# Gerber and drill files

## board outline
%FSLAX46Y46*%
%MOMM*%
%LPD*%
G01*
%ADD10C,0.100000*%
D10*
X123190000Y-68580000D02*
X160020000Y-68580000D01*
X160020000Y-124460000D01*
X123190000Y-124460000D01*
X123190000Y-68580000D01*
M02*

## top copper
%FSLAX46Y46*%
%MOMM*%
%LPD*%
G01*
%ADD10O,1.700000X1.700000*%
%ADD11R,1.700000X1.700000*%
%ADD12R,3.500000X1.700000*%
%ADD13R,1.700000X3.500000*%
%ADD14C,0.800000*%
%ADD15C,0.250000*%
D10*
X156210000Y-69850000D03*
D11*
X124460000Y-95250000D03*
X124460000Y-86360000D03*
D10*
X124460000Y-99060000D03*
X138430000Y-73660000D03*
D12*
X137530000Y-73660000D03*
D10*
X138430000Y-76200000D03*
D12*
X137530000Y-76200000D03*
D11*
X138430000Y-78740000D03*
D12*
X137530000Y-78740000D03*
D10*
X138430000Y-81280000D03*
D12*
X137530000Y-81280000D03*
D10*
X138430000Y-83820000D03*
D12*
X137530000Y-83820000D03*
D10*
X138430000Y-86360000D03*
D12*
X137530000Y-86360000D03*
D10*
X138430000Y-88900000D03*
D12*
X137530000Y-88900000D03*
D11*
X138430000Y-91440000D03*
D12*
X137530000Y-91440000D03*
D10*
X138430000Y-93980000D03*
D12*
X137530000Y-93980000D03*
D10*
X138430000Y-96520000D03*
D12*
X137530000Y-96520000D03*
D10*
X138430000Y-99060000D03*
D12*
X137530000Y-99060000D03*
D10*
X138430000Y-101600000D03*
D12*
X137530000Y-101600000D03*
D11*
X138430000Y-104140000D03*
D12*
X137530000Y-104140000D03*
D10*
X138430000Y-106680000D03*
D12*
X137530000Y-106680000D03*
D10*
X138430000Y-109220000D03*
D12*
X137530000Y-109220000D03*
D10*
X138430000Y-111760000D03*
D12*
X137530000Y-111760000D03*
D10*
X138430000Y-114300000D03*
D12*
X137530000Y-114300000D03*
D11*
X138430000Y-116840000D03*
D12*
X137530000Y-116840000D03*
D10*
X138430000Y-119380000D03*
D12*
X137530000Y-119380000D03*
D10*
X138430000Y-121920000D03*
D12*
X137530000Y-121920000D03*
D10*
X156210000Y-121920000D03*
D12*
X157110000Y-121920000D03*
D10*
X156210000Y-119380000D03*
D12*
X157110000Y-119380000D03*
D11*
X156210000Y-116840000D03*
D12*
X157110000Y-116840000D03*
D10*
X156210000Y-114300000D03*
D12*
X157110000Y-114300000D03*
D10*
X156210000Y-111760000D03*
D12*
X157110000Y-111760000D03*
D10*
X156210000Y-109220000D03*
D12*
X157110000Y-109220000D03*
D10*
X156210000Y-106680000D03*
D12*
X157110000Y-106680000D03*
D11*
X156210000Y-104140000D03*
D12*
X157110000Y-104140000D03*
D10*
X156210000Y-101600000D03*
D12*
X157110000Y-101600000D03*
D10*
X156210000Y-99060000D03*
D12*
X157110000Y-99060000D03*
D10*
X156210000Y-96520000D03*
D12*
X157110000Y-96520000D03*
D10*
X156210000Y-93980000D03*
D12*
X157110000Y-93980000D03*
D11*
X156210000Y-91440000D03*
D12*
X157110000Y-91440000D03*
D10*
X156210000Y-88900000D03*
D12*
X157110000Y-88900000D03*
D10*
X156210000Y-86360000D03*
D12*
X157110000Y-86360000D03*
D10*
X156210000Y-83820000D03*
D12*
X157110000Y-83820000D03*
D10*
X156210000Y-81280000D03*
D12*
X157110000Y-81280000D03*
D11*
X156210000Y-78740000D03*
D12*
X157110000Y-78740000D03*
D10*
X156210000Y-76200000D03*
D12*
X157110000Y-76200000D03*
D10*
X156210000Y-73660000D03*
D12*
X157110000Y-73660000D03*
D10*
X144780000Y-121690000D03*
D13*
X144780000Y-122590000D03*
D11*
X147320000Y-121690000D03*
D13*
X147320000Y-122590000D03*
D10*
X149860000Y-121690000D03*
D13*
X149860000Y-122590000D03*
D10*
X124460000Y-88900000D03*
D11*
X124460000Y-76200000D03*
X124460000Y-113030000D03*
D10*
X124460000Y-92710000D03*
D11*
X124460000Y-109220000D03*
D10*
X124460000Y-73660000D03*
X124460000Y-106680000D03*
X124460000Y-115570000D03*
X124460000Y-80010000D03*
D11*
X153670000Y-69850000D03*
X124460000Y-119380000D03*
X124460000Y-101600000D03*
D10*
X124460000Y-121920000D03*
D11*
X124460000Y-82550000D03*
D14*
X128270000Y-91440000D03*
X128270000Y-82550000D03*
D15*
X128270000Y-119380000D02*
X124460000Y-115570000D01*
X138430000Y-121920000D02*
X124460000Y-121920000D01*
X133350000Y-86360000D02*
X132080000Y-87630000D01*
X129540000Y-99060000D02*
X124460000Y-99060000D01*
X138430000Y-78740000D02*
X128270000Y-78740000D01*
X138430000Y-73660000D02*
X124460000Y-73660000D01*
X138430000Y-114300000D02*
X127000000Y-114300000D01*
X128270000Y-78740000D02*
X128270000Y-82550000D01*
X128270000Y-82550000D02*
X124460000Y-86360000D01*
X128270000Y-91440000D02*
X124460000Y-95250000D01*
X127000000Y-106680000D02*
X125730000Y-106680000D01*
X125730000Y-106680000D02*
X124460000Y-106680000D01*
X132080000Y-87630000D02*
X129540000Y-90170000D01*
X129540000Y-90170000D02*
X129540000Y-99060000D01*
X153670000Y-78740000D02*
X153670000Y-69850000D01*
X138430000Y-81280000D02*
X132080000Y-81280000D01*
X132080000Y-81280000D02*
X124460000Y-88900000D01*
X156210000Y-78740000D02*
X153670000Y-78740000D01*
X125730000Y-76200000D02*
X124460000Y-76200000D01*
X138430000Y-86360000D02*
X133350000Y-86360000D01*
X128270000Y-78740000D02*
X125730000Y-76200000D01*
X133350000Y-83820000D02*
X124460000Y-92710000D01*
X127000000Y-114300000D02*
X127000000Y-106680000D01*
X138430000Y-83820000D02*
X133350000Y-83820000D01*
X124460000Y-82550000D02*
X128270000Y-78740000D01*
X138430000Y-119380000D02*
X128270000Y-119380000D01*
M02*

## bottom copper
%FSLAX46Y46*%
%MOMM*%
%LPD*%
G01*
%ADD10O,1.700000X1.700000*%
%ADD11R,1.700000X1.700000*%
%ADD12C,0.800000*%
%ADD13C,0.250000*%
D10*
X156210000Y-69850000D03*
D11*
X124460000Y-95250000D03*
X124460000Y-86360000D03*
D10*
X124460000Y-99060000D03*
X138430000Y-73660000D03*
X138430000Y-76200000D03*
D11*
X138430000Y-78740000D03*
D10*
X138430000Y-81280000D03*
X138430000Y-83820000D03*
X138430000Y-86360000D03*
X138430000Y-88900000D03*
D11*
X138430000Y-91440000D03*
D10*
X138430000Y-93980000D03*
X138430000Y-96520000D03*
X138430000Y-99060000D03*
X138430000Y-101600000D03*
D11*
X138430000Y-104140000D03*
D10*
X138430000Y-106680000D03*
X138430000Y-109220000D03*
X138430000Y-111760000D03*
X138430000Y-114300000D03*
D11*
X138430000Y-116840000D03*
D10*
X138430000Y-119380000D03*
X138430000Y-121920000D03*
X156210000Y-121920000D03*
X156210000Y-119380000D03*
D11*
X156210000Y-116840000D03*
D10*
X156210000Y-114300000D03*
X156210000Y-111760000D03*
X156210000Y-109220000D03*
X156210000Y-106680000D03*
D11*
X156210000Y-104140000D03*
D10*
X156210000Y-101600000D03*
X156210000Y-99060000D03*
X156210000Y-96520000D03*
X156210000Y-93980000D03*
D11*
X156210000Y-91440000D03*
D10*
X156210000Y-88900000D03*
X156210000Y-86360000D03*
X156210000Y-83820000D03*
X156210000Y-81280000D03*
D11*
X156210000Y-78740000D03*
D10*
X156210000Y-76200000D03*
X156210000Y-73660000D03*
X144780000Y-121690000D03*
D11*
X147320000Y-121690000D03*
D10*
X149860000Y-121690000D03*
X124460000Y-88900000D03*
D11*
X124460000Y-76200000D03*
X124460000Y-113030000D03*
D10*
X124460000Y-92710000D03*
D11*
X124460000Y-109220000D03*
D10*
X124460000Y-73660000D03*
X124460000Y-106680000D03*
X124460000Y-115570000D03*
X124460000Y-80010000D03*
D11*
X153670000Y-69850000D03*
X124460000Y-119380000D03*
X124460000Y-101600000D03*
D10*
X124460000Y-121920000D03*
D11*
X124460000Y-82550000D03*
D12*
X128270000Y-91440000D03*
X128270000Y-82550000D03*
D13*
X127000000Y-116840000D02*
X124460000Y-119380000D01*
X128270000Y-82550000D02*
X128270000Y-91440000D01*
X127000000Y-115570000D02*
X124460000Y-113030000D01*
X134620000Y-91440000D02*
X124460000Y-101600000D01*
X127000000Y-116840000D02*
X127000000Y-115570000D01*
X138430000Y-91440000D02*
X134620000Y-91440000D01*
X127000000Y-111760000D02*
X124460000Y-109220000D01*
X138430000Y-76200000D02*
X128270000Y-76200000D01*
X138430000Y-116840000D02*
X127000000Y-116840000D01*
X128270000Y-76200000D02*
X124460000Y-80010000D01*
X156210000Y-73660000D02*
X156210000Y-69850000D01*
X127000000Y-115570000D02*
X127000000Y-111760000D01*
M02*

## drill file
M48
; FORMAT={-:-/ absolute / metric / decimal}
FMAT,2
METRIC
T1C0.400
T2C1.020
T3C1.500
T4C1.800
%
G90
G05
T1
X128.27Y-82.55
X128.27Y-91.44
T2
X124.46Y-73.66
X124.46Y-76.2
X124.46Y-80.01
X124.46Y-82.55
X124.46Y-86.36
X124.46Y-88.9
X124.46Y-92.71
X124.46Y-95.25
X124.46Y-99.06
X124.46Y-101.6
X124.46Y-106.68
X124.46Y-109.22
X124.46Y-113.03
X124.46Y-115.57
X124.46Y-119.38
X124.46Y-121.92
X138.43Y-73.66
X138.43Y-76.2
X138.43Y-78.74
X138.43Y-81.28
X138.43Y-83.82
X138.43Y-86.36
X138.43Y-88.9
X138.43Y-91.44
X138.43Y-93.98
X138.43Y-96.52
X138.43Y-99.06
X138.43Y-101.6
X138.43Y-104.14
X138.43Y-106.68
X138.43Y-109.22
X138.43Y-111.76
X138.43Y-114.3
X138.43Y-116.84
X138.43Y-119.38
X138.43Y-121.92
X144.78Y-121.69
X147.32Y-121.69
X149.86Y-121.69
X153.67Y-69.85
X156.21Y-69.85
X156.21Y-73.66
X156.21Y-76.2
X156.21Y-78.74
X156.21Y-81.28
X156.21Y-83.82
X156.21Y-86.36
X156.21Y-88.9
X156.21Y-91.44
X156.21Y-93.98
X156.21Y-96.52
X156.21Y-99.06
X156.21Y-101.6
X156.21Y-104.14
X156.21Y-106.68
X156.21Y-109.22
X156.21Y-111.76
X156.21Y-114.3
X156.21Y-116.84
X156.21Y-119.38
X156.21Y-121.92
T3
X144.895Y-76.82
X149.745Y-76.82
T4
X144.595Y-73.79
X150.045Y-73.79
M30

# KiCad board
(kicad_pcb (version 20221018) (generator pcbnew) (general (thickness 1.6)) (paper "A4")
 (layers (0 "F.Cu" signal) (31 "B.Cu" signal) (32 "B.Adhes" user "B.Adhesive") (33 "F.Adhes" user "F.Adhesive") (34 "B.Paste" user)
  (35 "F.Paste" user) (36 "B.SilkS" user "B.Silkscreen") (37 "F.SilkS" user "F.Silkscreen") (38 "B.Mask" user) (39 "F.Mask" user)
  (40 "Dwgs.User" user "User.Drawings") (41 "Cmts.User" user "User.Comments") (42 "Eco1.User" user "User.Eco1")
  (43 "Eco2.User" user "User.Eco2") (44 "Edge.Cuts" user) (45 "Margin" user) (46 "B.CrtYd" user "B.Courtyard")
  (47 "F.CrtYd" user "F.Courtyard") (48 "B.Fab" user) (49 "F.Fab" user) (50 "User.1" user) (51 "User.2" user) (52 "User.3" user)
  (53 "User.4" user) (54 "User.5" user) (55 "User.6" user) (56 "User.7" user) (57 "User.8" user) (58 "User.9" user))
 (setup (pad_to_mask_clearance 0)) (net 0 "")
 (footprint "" (layer "F.Cu") (at 156.21 69.85)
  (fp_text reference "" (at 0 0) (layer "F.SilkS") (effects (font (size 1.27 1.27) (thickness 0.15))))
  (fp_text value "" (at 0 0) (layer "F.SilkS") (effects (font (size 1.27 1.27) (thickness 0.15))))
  (pad "39" thru_hole oval (at 0 0) (size 1.7 1.7) (drill 1.02) (layers "*.Cu" "*.Mask")))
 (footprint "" (layer "F.Cu") (at 124.46 95.25)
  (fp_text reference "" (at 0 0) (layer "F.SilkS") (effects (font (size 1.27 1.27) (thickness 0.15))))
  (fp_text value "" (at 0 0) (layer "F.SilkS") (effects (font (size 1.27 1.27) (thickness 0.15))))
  (pad "3" thru_hole rect (at 0 0) (size 1.7 1.7) (drill 1.02) (layers "*.Cu" "*.Mask")))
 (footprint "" (layer "F.Cu") (at 124.46 86.36)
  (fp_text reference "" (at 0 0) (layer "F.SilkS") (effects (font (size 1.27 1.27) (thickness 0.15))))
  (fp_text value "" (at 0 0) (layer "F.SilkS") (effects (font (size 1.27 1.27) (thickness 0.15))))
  (pad "3" thru_hole rect (at 0 0) (size 1.7 1.7) (drill 1.02) (layers "*.Cu" "*.Mask")))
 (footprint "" (layer "F.Cu") (at 124.46 99.06)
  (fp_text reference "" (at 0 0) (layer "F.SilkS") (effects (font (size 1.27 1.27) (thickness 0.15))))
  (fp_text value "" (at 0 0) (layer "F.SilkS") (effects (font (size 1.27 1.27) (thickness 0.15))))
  (pad "6" thru_hole oval (at 0 0) (size 1.7 1.7) (drill 1.02) (layers "*.Cu" "*.Mask")))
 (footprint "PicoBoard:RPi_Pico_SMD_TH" (layer "F.Cu") (at 147.32 97.79)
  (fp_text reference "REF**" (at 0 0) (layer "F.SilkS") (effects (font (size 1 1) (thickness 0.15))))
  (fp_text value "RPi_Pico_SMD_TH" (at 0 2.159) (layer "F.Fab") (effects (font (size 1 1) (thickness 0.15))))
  (pad "" np_thru_hole oval (at -2.725 -24) (size 1.8 1.8) (drill 1.8) (layers "*.Cu" "*.Mask"))
  (pad "" np_thru_hole oval (at -2.425 -20.97) (size 1.5 1.5) (drill 1.5) (layers "*.Cu" "*.Mask"))
  (pad "" np_thru_hole oval (at 2.425 -20.97) (size 1.5 1.5) (drill 1.5) (layers "*.Cu" "*.Mask"))
  (pad "" np_thru_hole oval (at 2.725 -24) (size 1.8 1.8) (drill 1.8) (layers "*.Cu" "*.Mask"))
  (pad "1" thru_hole oval (at -8.89 -24.13) (size 1.7 1.7) (drill 1.02) (layers "*.Cu" "*.Mask"))
  (pad "1" smd rect (at -8.89 -24.13) (size 3.5 1.7) (drill (offset -0.9 0)) (layers "F.Cu" "F.Mask"))
  (pad "2" thru_hole oval (at -8.89 -21.59) (size 1.7 1.7) (drill 1.02) (layers "*.Cu" "*.Mask"))
  (pad "2" smd rect (at -8.89 -21.59) (size 3.5 1.7) (drill (offset -0.9 0)) (layers "F.Cu" "F.Mask"))
  (pad "3" thru_hole rect (at -8.89 -19.05) (size 1.7 1.7) (drill 1.02) (layers "*.Cu" "*.Mask"))
  (pad "3" smd rect (at -8.89 -19.05) (size 3.5 1.7) (drill (offset -0.9 0)) (layers "F.Cu" "F.Mask"))
  (pad "4" thru_hole oval (at -8.89 -16.51) (size 1.7 1.7) (drill 1.02) (layers "*.Cu" "*.Mask"))
  (pad "4" smd rect (at -8.89 -16.51) (size 3.5 1.7) (drill (offset -0.9 0)) (layers "F.Cu" "F.Mask"))
  (pad "5" thru_hole oval (at -8.89 -13.97) (size 1.7 1.7) (drill 1.02) (layers "*.Cu" "*.Mask"))
  (pad "5" smd rect (at -8.89 -13.97) (size 3.5 1.7) (drill (offset -0.9 0)) (layers "F.Cu" "F.Mask"))
  (pad "6" thru_hole oval (at -8.89 -11.43) (size 1.7 1.7) (drill 1.02) (layers "*.Cu" "*.Mask"))
  (pad "6" smd rect (at -8.89 -11.43) (size 3.5 1.7) (drill (offset -0.9 0)) (layers "F.Cu" "F.Mask"))
  (pad "7" thru_hole oval (at -8.89 -8.89) (size 1.7 1.7) (drill 1.02) (layers "*.Cu" "*.Mask"))
  (pad "7" smd rect (at -8.89 -8.89) (size 3.5 1.7) (drill (offset -0.9 0)) (layers "F.Cu" "F.Mask"))
  (pad "8" thru_hole rect (at -8.89 -6.35) (size 1.7 1.7) (drill 1.02) (layers "*.Cu" "*.Mask"))
  (pad "8" smd rect (at -8.89 -6.35) (size 3.5 1.7) (drill (offset -0.9 0)) (layers "F.Cu" "F.Mask"))
  (pad "9" thru_hole oval (at -8.89 -3.81) (size 1.7 1.7) (drill 1.02) (layers "*.Cu" "*.Mask"))
  (pad "9" smd rect (at -8.89 -3.81) (size 3.5 1.7) (drill (offset -0.9 0)) (layers "F.Cu" "F.Mask"))
  (pad "10" thru_hole oval (at -8.89 -1.27) (size 1.7 1.7) (drill 1.02) (layers "*.Cu" "*.Mask"))
  (pad "10" smd rect (at -8.89 -1.27) (size 3.5 1.7) (drill (offset -0.9 0)) (layers "F.Cu" "F.Mask"))
  (pad "11" thru_hole oval (at -8.89 1.27) (size 1.7 1.7) (drill 1.02) (layers "*.Cu" "*.Mask"))
  (pad "11" smd rect (at -8.89 1.27) (size 3.5 1.7) (drill (offset -0.9 0)) (layers "F.Cu" "F.Mask"))
  (pad "12" thru_hole oval (at -8.89 3.81) (size 1.7 1.7) (drill 1.02) (layers "*.Cu" "*.Mask"))
  (pad "12" smd rect (at -8.89 3.81) (size 3.5 1.7) (drill (offset -0.9 0)) (layers "F.Cu" "F.Mask"))
  (pad "13" thru_hole rect (at -8.89 6.35) (size 1.7 1.7) (drill 1.02) (layers "*.Cu" "*.Mask"))
  (pad "13" smd rect (at -8.89 6.35) (size 3.5 1.7) (drill (offset -0.9 0)) (layers "F.Cu" "F.Mask"))
  (pad "14" thru_hole oval (at -8.89 8.89) (size 1.7 1.7) (drill 1.02) (layers "*.Cu" "*.Mask"))
  (pad "14" smd rect (at -8.89 8.89) (size 3.5 1.7) (drill (offset -0.9 0)) (layers "F.Cu" "F.Mask"))
  (pad "15" thru_hole oval (at -8.89 11.43) (size 1.7 1.7) (drill 1.02) (layers "*.Cu" "*.Mask"))
  (pad "15" smd rect (at -8.89 11.43) (size 3.5 1.7) (drill (offset -0.9 0)) (layers "F.Cu" "F.Mask"))
  (pad "16" thru_hole oval (at -8.89 13.97) (size 1.7 1.7) (drill 1.02) (layers "*.Cu" "*.Mask"))
  (pad "16" smd rect (at -8.89 13.97) (size 3.5 1.7) (drill (offset -0.9 0)) (layers "F.Cu" "F.Mask"))
  (pad "17" thru_hole oval (at -8.89 16.51) (size 1.7 1.7) (drill 1.02) (layers "*.Cu" "*.Mask"))
  (pad "17" smd rect (at -8.89 16.51) (size 3.5 1.7) (drill (offset -0.9 0)) (layers "F.Cu" "F.Mask"))
  (pad "18" thru_hole rect (at -8.89 19.05) (size 1.7 1.7) (drill 1.02) (layers "*.Cu" "*.Mask"))
  (pad "18" smd rect (at -8.89 19.05) (size 3.5 1.7) (drill (offset -0.9 0)) (layers "F.Cu" "F.Mask"))
  (pad "19" thru_hole oval (at -8.89 21.59) (size 1.7 1.7) (drill 1.02) (layers "*.Cu" "*.Mask"))
  (pad "19" smd rect (at -8.89 21.59) (size 3.5 1.7) (drill (offset -0.9 0)) (layers "F.Cu" "F.Mask"))
  (pad "20" thru_hole oval (at -8.89 24.13) (size 1.7 1.7) (drill 1.02) (layers "*.Cu" "*.Mask"))
  (pad "20" smd rect (at -8.89 24.13) (size 3.5 1.7) (drill (offset -0.9 0)) (layers "F.Cu" "F.Mask"))
  (pad "21" thru_hole oval (at 8.89 24.13) (size 1.7 1.7) (drill 1.02) (layers "*.Cu" "*.Mask"))
  (pad "21" smd rect (at 8.89 24.13) (size 3.5 1.7) (drill (offset 0.9 0)) (layers "F.Cu" "F.Mask"))
  (pad "22" thru_hole oval (at 8.89 21.59) (size 1.7 1.7) (drill 1.02) (layers "*.Cu" "*.Mask"))
  (pad "22" smd rect (at 8.89 21.59) (size 3.5 1.7) (drill (offset 0.9 0)) (layers "F.Cu" "F.Mask"))
  (pad "23" thru_hole rect (at 8.89 19.05) (size 1.7 1.7) (drill 1.02) (layers "*.Cu" "*.Mask"))
  (pad "23" smd rect (at 8.89 19.05) (size 3.5 1.7) (drill (offset 0.9 0)) (layers "F.Cu" "F.Mask"))
  (pad "24" thru_hole oval (at 8.89 16.51) (size 1.7 1.7) (drill 1.02) (layers "*.Cu" "*.Mask"))
  (pad "24" smd rect (at 8.89 16.51) (size 3.5 1.7) (drill (offset 0.9 0)) (layers "F.Cu" "F.Mask"))
  (pad "25" thru_hole oval (at 8.89 13.97) (size 1.7 1.7) (drill 1.02) (layers "*.Cu" "*.Mask"))
  (pad "25" smd rect (at 8.89 13.97) (size 3.5 1.7) (drill (offset 0.9 0)) (layers "F.Cu" "F.Mask"))
  (pad "26" thru_hole oval (at 8.89 11.43) (size 1.7 1.7) (drill 1.02) (layers "*.Cu" "*.Mask"))
  (pad "26" smd rect (at 8.89 11.43) (size 3.5 1.7) (drill (offset 0.9 0)) (layers "F.Cu" "F.Mask"))
  (pad "27" thru_hole oval (at 8.89 8.89) (size 1.7 1.7) (drill 1.02) (layers "*.Cu" "*.Mask"))
  (pad "27" smd rect (at 8.89 8.89) (size 3.5 1.7) (drill (offset 0.9 0)) (layers "F.Cu" "F.Mask"))
  (pad "28" thru_hole rect (at 8.89 6.35) (size 1.7 1.7) (drill 1.02) (layers "*.Cu" "*.Mask"))
  (pad "28" smd rect (at 8.89 6.35) (size 3.5 1.7) (drill (offset 0.9 0)) (layers "F.Cu" "F.Mask"))
  (pad "29" thru_hole oval (at 8.89 3.81) (size 1.7 1.7) (drill 1.02) (layers "*.Cu" "*.Mask"))
  (pad "29" smd rect (at 8.89 3.81) (size 3.5 1.7) (drill (offset 0.9 0)) (layers "F.Cu" "F.Mask"))
  (pad "30" thru_hole oval (at 8.89 1.27) (size 1.7 1.7) (drill 1.02) (layers "*.Cu" "*.Mask"))
  (pad "30" smd rect (at 8.89 1.27) (size 3.5 1.7) (drill (offset 0.9 0)) (layers "F.Cu" "F.Mask"))
  (pad "31" thru_hole oval (at 8.89 -1.27) (size 1.7 1.7) (drill 1.02) (layers "*.Cu" "*.Mask"))
  (pad "31" smd rect (at 8.89 -1.27) (size 3.5 1.7) (drill (offset 0.9 0)) (layers "F.Cu" "F.Mask"))
  (pad "32" thru_hole oval (at 8.89 -3.81) (size 1.7 1.7) (drill 1.02) (layers "*.Cu" "*.Mask"))
  (pad "32" smd rect (at 8.89 -3.81) (size 3.5 1.7) (drill (offset 0.9 0)) (layers "F.Cu" "F.Mask"))
  (pad "33" thru_hole rect (at 8.89 -6.35) (size 1.7 1.7) (drill 1.02) (layers "*.Cu" "*.Mask"))
  (pad "33" smd rect (at 8.89 -6.35) (size 3.5 1.7) (drill (offset 0.9 0)) (layers "F.Cu" "F.Mask"))
  (pad "34" thru_hole oval (at 8.89 -8.89) (size 1.7 1.7) (drill 1.02) (layers "*.Cu" "*.Mask"))
  (pad "34" smd rect (at 8.89 -8.89) (size 3.5 1.7) (drill (offset 0.9 0)) (layers "F.Cu" "F.Mask"))
  (pad "35" thru_hole oval (at 8.89 -11.43) (size 1.7 1.7) (drill 1.02) (layers "*.Cu" "*.Mask"))
  (pad "35" smd rect (at 8.89 -11.43) (size 3.5 1.7) (drill (offset 0.9 0)) (layers "F.Cu" "F.Mask"))
  (pad "36" thru_hole oval (at 8.89 -13.97) (size 1.7 1.7) (drill 1.02) (layers "*.Cu" "*.Mask"))
  (pad "36" smd rect (at 8.89 -13.97) (size 3.5 1.7) (drill (offset 0.9 0)) (layers "F.Cu" "F.Mask"))
  (pad "37" thru_hole oval (at 8.89 -16.51) (size 1.7 1.7) (drill 1.02) (layers "*.Cu" "*.Mask"))
  (pad "37" smd rect (at 8.89 -16.51) (size 3.5 1.7) (drill (offset 0.9 0)) (layers "F.Cu" "F.Mask"))
  (pad "38" thru_hole rect (at 8.89 -19.05) (size 1.7 1.7) (drill 1.02) (layers "*.Cu" "*.Mask"))
  (pad "38" smd rect (at 8.89 -19.05) (size 3.5 1.7) (drill (offset 0.9 0)) (layers "F.Cu" "F.Mask"))
  (pad "39" thru_hole oval (at 8.89 -21.59) (size 1.7 1.7) (drill 1.02) (layers "*.Cu" "*.Mask"))
  (pad "39" smd rect (at 8.89 -21.59) (size 3.5 1.7) (drill (offset 0.9 0)) (layers "F.Cu" "F.Mask"))
  (pad "40" thru_hole oval (at 8.89 -24.13) (size 1.7 1.7) (drill 1.02) (layers "*.Cu" "*.Mask"))
  (pad "40" smd rect (at 8.89 -24.13) (size 3.5 1.7) (drill (offset 0.9 0)) (layers "F.Cu" "F.Mask"))
  (pad "41" thru_hole oval (at -2.54 23.9) (size 1.7 1.7) (drill 1.02) (layers "*.Cu" "*.Mask"))
  (pad "41" smd rect (at -2.54 23.9 90) (size 3.5 1.7) (drill (offset -0.9 0)) (layers "F.Cu" "F.Mask"))
  (pad "42" thru_hole rect (at 0 23.9) (size 1.7 1.7) (drill 1.02) (layers "*.Cu" "*.Mask"))
  (pad "42" smd rect (at 0 23.9 90) (size 3.5 1.7) (drill (offset -0.9 0)) (layers "F.Cu" "F.Mask"))
  (pad "43" thru_hole oval (at 2.54 23.9) (size 1.7 1.7) (drill 1.02) (layers "*.Cu" "*.Mask"))
  (pad "43" smd rect (at 2.54 23.9 90) (size 3.5 1.7) (drill (offset -0.9 0)) (layers "F.Cu" "F.Mask")))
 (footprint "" (layer "F.Cu") (at 124.46 88.9)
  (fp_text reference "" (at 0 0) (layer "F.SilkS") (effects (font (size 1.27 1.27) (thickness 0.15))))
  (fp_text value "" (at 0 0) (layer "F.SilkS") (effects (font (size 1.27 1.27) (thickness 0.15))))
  (pad "4" thru_hole oval (at 0 0) (size 1.7 1.7) (drill 1.02) (layers "*.Cu" "*.Mask")))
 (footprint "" (layer "F.Cu") (at 124.46 76.2)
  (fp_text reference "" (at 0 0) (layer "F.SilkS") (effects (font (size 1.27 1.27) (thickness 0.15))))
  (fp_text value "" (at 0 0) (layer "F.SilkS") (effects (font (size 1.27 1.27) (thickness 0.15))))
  (pad "3" thru_hole rect (at 0 0) (size 1.7 1.7) (drill 1.02) (layers "*.Cu" "*.Mask")))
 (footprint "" (layer "F.Cu") (at 124.46 113.03)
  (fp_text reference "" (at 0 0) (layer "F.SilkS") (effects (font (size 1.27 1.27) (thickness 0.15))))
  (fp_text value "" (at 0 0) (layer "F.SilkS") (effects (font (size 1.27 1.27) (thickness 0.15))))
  (pad "18" thru_hole rect (at 0 0) (size 1.7 1.7) (drill 1.02) (layers "*.Cu" "*.Mask")))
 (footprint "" (layer "F.Cu") (at 124.46 92.71)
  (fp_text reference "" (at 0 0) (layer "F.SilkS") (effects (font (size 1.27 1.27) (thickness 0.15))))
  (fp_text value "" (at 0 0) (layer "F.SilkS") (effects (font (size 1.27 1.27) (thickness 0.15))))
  (pad "5" thru_hole oval (at 0 0) (size 1.7 1.7) (drill 1.02) (layers "*.Cu" "*.Mask")))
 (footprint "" (layer "F.Cu") (at 124.46 109.22)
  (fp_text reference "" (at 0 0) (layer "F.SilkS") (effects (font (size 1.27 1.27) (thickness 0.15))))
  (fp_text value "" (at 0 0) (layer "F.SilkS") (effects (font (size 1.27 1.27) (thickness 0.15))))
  (pad "18" thru_hole rect (at 0 0) (size 1.7 1.7) (drill 1.02) (layers "*.Cu" "*.Mask")))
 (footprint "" (layer "F.Cu") (at 124.46 73.66)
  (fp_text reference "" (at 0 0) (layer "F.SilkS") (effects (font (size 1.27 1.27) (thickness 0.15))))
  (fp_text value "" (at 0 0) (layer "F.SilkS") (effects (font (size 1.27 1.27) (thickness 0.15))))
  (pad "1" thru_hole oval (at 0 0) (size 1.7 1.7) (drill 1.02) (layers "*.Cu" "*.Mask")))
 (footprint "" (layer "F.Cu") (at 124.46 106.68)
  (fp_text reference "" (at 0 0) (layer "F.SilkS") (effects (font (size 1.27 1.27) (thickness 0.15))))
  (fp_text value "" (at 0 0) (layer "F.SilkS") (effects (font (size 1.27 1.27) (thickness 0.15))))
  (pad "17" thru_hole oval (at 0 0) (size 1.7 1.7) (drill 1.02) (layers "*.Cu" "*.Mask")))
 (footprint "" (layer "F.Cu") (at 124.46 115.57)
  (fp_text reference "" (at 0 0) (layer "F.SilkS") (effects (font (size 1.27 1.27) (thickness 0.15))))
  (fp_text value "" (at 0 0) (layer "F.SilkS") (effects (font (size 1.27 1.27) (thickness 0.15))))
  (pad "19" thru_hole oval (at 0 0) (size 1.7 1.7) (drill 1.02) (layers "*.Cu" "*.Mask")))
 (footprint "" (layer "F.Cu") (at 124.46 80.01)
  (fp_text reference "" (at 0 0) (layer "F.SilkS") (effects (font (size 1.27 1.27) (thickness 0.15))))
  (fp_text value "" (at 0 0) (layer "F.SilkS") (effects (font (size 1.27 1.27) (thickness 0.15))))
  (pad "2" thru_hole oval (at 0 0) (size 1.7 1.7) (drill 1.02) (layers "*.Cu" "*.Mask")))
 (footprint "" (layer "F.Cu") (at 153.67 69.85)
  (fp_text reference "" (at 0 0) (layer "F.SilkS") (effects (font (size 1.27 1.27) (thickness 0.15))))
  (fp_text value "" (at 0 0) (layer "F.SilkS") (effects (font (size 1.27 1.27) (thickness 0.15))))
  (pad "38" thru_hole rect (at 0 0) (size 1.7 1.7) (drill 1.02) (layers "*.Cu" "*.Mask")))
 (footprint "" (layer "F.Cu") (at 124.46 119.38)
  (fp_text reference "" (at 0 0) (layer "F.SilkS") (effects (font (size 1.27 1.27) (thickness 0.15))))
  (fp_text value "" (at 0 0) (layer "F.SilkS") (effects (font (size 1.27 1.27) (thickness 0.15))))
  (pad "18" thru_hole rect (at 0 0) (size 1.7 1.7) (drill 1.02) (layers "*.Cu" "*.Mask")))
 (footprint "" (layer "F.Cu") (at 124.46 101.6)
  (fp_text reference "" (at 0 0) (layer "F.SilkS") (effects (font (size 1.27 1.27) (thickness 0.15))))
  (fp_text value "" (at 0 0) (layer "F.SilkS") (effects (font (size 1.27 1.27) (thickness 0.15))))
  (pad "8" thru_hole rect (at 0 0) (size 1.7 1.7) (drill 1.02) (layers "*.Cu" "*.Mask")))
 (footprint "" (layer "F.Cu") (at 124.46 121.92)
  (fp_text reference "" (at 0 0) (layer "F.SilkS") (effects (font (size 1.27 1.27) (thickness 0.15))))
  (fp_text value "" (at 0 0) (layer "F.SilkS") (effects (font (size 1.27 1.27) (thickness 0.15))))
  (pad "20" thru_hole oval (at 0 0) (size 1.7 1.7) (drill 1.02) (layers "*.Cu" "*.Mask")))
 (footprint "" (layer "F.Cu") (at 124.46 82.55)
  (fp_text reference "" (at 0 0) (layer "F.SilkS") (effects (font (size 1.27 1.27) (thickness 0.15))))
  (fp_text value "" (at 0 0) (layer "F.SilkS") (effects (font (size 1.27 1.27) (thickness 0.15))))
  (pad "3" thru_hole rect (at 0 0) (size 1.7 1.7) (drill 1.02) (layers "*.Cu" "*.Mask")))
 (gr_rect (start 123.19 68.58) (end 160.02 124.46) (stroke (width 0.1) (type default)) (fill none) (layer "Edge.Cuts"))
 (segment (start 128.27 119.38) (end 124.46 115.57) (width 0.25) (layer "F.Cu") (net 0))
 (segment (start 138.43 121.92) (end 124.46 121.92) (width 0.25) (layer "F.Cu") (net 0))
 (segment (start 133.35 86.36) (end 132.08 87.63) (width 0.25) (layer "F.Cu") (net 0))
 (segment (start 129.54 99.06) (end 124.46 99.06) (width 0.25) (layer "F.Cu") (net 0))
 (segment (start 138.43 78.74) (end 128.27 78.74) (width 0.25) (layer "F.Cu") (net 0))
 (segment (start 138.43 73.66) (end 124.46 73.66) (width 0.25) (layer "F.Cu") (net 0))
 (segment (start 138.43 114.3) (end 127 114.3) (width 0.25) (layer "F.Cu") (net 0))
 (segment (start 128.27 78.74) (end 128.27 82.55) (width 0.25) (layer "F.Cu") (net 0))
 (segment (start 128.27 82.55) (end 124.46 86.36) (width 0.25) (layer "F.Cu") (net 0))
 (segment (start 128.27 91.44) (end 124.46 95.25) (width 0.25) (layer "F.Cu") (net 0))
 (segment (start 127 106.68) (end 125.73 106.68) (width 0.25) (layer "F.Cu") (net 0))
 (segment (start 125.73 106.68) (end 124.46 106.68) (width 0.25) (layer "F.Cu") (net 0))
 (segment (start 132.08 87.63) (end 129.54 90.17) (width 0.25) (layer "F.Cu") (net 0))
 (segment (start 129.54 90.17) (end 129.54 99.06) (width 0.25) (layer "F.Cu") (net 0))
 (segment (start 153.67 78.74) (end 153.67 69.85) (width 0.25) (layer "F.Cu") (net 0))
 (segment (start 138.43 81.28) (end 132.08 81.28) (width 0.25) (layer "F.Cu") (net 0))
 (segment (start 132.08 81.28) (end 124.46 88.9) (width 0.25) (layer "F.Cu") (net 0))
 (segment (start 156.21 78.74) (end 153.67 78.74) (width 0.25) (layer "F.Cu") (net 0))
 (segment (start 125.73 76.2) (end 124.46 76.2) (width 0.25) (layer "F.Cu") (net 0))
 (segment (start 138.43 86.36) (end 133.35 86.36) (width 0.25) (layer "F.Cu") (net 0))
 (segment (start 128.27 78.74) (end 125.73 76.2) (width 0.25) (layer "F.Cu") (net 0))
 (segment (start 133.35 83.82) (end 124.46 92.71) (width 0.25) (layer "F.Cu") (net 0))
 (segment (start 127 114.3) (end 127 106.68) (width 0.25) (layer "F.Cu") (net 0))
 (segment (start 138.43 83.82) (end 133.35 83.82) (width 0.25) (layer "F.Cu") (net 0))
 (segment (start 124.46 82.55) (end 128.27 78.74) (width 0.25) (layer "F.Cu") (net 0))
 (segment (start 138.43 119.38) (end 128.27 119.38) (width 0.25) (layer "F.Cu") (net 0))
 (via (at 128.27 91.44) (size 0.8) (drill 0.4) (layers "F.Cu" "B.Cu") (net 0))
 (via (at 128.27 82.55) (size 0.8) (drill 0.4) (layers "F.Cu" "B.Cu") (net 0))
 (segment (start 127 116.84) (end 124.46 119.38) (width 0.25) (layer "B.Cu") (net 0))
 (segment (start 128.27 82.55) (end 128.27 91.44) (width 0.25) (layer "B.Cu") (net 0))
 (segment (start 127 115.57) (end 124.46 113.03) (width 0.25) (layer "B.Cu") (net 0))
 (segment (start 134.62 91.44) (end 124.46 101.6) (width 0.25) (layer "B.Cu") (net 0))
 (segment (start 127 116.84) (end 127 115.57) (width 0.25) (layer "B.Cu") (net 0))
 (segment (start 138.43 91.44) (end 134.62 91.44) (width 0.25) (layer "B.Cu") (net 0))
 (segment (start 127 111.76) (end 124.46 109.22) (width 0.25) (layer "B.Cu") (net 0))
 (segment (start 138.43 76.2) (end 128.27 76.2) (width 0.25) (layer "B.Cu") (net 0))
 (segment (start 138.43 116.84) (end 127 116.84) (width 0.25) (layer "B.Cu") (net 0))
 (segment (start 128.27 76.2) (end 124.46 80.01) (width 0.25) (layer "B.Cu") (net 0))
 (segment (start 156.21 73.66) (end 156.21 69.85) (width 0.25) (layer "B.Cu") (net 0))
 (segment (start 127 115.57) (end 127 111.76) (width 0.25) (layer "B.Cu") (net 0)))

